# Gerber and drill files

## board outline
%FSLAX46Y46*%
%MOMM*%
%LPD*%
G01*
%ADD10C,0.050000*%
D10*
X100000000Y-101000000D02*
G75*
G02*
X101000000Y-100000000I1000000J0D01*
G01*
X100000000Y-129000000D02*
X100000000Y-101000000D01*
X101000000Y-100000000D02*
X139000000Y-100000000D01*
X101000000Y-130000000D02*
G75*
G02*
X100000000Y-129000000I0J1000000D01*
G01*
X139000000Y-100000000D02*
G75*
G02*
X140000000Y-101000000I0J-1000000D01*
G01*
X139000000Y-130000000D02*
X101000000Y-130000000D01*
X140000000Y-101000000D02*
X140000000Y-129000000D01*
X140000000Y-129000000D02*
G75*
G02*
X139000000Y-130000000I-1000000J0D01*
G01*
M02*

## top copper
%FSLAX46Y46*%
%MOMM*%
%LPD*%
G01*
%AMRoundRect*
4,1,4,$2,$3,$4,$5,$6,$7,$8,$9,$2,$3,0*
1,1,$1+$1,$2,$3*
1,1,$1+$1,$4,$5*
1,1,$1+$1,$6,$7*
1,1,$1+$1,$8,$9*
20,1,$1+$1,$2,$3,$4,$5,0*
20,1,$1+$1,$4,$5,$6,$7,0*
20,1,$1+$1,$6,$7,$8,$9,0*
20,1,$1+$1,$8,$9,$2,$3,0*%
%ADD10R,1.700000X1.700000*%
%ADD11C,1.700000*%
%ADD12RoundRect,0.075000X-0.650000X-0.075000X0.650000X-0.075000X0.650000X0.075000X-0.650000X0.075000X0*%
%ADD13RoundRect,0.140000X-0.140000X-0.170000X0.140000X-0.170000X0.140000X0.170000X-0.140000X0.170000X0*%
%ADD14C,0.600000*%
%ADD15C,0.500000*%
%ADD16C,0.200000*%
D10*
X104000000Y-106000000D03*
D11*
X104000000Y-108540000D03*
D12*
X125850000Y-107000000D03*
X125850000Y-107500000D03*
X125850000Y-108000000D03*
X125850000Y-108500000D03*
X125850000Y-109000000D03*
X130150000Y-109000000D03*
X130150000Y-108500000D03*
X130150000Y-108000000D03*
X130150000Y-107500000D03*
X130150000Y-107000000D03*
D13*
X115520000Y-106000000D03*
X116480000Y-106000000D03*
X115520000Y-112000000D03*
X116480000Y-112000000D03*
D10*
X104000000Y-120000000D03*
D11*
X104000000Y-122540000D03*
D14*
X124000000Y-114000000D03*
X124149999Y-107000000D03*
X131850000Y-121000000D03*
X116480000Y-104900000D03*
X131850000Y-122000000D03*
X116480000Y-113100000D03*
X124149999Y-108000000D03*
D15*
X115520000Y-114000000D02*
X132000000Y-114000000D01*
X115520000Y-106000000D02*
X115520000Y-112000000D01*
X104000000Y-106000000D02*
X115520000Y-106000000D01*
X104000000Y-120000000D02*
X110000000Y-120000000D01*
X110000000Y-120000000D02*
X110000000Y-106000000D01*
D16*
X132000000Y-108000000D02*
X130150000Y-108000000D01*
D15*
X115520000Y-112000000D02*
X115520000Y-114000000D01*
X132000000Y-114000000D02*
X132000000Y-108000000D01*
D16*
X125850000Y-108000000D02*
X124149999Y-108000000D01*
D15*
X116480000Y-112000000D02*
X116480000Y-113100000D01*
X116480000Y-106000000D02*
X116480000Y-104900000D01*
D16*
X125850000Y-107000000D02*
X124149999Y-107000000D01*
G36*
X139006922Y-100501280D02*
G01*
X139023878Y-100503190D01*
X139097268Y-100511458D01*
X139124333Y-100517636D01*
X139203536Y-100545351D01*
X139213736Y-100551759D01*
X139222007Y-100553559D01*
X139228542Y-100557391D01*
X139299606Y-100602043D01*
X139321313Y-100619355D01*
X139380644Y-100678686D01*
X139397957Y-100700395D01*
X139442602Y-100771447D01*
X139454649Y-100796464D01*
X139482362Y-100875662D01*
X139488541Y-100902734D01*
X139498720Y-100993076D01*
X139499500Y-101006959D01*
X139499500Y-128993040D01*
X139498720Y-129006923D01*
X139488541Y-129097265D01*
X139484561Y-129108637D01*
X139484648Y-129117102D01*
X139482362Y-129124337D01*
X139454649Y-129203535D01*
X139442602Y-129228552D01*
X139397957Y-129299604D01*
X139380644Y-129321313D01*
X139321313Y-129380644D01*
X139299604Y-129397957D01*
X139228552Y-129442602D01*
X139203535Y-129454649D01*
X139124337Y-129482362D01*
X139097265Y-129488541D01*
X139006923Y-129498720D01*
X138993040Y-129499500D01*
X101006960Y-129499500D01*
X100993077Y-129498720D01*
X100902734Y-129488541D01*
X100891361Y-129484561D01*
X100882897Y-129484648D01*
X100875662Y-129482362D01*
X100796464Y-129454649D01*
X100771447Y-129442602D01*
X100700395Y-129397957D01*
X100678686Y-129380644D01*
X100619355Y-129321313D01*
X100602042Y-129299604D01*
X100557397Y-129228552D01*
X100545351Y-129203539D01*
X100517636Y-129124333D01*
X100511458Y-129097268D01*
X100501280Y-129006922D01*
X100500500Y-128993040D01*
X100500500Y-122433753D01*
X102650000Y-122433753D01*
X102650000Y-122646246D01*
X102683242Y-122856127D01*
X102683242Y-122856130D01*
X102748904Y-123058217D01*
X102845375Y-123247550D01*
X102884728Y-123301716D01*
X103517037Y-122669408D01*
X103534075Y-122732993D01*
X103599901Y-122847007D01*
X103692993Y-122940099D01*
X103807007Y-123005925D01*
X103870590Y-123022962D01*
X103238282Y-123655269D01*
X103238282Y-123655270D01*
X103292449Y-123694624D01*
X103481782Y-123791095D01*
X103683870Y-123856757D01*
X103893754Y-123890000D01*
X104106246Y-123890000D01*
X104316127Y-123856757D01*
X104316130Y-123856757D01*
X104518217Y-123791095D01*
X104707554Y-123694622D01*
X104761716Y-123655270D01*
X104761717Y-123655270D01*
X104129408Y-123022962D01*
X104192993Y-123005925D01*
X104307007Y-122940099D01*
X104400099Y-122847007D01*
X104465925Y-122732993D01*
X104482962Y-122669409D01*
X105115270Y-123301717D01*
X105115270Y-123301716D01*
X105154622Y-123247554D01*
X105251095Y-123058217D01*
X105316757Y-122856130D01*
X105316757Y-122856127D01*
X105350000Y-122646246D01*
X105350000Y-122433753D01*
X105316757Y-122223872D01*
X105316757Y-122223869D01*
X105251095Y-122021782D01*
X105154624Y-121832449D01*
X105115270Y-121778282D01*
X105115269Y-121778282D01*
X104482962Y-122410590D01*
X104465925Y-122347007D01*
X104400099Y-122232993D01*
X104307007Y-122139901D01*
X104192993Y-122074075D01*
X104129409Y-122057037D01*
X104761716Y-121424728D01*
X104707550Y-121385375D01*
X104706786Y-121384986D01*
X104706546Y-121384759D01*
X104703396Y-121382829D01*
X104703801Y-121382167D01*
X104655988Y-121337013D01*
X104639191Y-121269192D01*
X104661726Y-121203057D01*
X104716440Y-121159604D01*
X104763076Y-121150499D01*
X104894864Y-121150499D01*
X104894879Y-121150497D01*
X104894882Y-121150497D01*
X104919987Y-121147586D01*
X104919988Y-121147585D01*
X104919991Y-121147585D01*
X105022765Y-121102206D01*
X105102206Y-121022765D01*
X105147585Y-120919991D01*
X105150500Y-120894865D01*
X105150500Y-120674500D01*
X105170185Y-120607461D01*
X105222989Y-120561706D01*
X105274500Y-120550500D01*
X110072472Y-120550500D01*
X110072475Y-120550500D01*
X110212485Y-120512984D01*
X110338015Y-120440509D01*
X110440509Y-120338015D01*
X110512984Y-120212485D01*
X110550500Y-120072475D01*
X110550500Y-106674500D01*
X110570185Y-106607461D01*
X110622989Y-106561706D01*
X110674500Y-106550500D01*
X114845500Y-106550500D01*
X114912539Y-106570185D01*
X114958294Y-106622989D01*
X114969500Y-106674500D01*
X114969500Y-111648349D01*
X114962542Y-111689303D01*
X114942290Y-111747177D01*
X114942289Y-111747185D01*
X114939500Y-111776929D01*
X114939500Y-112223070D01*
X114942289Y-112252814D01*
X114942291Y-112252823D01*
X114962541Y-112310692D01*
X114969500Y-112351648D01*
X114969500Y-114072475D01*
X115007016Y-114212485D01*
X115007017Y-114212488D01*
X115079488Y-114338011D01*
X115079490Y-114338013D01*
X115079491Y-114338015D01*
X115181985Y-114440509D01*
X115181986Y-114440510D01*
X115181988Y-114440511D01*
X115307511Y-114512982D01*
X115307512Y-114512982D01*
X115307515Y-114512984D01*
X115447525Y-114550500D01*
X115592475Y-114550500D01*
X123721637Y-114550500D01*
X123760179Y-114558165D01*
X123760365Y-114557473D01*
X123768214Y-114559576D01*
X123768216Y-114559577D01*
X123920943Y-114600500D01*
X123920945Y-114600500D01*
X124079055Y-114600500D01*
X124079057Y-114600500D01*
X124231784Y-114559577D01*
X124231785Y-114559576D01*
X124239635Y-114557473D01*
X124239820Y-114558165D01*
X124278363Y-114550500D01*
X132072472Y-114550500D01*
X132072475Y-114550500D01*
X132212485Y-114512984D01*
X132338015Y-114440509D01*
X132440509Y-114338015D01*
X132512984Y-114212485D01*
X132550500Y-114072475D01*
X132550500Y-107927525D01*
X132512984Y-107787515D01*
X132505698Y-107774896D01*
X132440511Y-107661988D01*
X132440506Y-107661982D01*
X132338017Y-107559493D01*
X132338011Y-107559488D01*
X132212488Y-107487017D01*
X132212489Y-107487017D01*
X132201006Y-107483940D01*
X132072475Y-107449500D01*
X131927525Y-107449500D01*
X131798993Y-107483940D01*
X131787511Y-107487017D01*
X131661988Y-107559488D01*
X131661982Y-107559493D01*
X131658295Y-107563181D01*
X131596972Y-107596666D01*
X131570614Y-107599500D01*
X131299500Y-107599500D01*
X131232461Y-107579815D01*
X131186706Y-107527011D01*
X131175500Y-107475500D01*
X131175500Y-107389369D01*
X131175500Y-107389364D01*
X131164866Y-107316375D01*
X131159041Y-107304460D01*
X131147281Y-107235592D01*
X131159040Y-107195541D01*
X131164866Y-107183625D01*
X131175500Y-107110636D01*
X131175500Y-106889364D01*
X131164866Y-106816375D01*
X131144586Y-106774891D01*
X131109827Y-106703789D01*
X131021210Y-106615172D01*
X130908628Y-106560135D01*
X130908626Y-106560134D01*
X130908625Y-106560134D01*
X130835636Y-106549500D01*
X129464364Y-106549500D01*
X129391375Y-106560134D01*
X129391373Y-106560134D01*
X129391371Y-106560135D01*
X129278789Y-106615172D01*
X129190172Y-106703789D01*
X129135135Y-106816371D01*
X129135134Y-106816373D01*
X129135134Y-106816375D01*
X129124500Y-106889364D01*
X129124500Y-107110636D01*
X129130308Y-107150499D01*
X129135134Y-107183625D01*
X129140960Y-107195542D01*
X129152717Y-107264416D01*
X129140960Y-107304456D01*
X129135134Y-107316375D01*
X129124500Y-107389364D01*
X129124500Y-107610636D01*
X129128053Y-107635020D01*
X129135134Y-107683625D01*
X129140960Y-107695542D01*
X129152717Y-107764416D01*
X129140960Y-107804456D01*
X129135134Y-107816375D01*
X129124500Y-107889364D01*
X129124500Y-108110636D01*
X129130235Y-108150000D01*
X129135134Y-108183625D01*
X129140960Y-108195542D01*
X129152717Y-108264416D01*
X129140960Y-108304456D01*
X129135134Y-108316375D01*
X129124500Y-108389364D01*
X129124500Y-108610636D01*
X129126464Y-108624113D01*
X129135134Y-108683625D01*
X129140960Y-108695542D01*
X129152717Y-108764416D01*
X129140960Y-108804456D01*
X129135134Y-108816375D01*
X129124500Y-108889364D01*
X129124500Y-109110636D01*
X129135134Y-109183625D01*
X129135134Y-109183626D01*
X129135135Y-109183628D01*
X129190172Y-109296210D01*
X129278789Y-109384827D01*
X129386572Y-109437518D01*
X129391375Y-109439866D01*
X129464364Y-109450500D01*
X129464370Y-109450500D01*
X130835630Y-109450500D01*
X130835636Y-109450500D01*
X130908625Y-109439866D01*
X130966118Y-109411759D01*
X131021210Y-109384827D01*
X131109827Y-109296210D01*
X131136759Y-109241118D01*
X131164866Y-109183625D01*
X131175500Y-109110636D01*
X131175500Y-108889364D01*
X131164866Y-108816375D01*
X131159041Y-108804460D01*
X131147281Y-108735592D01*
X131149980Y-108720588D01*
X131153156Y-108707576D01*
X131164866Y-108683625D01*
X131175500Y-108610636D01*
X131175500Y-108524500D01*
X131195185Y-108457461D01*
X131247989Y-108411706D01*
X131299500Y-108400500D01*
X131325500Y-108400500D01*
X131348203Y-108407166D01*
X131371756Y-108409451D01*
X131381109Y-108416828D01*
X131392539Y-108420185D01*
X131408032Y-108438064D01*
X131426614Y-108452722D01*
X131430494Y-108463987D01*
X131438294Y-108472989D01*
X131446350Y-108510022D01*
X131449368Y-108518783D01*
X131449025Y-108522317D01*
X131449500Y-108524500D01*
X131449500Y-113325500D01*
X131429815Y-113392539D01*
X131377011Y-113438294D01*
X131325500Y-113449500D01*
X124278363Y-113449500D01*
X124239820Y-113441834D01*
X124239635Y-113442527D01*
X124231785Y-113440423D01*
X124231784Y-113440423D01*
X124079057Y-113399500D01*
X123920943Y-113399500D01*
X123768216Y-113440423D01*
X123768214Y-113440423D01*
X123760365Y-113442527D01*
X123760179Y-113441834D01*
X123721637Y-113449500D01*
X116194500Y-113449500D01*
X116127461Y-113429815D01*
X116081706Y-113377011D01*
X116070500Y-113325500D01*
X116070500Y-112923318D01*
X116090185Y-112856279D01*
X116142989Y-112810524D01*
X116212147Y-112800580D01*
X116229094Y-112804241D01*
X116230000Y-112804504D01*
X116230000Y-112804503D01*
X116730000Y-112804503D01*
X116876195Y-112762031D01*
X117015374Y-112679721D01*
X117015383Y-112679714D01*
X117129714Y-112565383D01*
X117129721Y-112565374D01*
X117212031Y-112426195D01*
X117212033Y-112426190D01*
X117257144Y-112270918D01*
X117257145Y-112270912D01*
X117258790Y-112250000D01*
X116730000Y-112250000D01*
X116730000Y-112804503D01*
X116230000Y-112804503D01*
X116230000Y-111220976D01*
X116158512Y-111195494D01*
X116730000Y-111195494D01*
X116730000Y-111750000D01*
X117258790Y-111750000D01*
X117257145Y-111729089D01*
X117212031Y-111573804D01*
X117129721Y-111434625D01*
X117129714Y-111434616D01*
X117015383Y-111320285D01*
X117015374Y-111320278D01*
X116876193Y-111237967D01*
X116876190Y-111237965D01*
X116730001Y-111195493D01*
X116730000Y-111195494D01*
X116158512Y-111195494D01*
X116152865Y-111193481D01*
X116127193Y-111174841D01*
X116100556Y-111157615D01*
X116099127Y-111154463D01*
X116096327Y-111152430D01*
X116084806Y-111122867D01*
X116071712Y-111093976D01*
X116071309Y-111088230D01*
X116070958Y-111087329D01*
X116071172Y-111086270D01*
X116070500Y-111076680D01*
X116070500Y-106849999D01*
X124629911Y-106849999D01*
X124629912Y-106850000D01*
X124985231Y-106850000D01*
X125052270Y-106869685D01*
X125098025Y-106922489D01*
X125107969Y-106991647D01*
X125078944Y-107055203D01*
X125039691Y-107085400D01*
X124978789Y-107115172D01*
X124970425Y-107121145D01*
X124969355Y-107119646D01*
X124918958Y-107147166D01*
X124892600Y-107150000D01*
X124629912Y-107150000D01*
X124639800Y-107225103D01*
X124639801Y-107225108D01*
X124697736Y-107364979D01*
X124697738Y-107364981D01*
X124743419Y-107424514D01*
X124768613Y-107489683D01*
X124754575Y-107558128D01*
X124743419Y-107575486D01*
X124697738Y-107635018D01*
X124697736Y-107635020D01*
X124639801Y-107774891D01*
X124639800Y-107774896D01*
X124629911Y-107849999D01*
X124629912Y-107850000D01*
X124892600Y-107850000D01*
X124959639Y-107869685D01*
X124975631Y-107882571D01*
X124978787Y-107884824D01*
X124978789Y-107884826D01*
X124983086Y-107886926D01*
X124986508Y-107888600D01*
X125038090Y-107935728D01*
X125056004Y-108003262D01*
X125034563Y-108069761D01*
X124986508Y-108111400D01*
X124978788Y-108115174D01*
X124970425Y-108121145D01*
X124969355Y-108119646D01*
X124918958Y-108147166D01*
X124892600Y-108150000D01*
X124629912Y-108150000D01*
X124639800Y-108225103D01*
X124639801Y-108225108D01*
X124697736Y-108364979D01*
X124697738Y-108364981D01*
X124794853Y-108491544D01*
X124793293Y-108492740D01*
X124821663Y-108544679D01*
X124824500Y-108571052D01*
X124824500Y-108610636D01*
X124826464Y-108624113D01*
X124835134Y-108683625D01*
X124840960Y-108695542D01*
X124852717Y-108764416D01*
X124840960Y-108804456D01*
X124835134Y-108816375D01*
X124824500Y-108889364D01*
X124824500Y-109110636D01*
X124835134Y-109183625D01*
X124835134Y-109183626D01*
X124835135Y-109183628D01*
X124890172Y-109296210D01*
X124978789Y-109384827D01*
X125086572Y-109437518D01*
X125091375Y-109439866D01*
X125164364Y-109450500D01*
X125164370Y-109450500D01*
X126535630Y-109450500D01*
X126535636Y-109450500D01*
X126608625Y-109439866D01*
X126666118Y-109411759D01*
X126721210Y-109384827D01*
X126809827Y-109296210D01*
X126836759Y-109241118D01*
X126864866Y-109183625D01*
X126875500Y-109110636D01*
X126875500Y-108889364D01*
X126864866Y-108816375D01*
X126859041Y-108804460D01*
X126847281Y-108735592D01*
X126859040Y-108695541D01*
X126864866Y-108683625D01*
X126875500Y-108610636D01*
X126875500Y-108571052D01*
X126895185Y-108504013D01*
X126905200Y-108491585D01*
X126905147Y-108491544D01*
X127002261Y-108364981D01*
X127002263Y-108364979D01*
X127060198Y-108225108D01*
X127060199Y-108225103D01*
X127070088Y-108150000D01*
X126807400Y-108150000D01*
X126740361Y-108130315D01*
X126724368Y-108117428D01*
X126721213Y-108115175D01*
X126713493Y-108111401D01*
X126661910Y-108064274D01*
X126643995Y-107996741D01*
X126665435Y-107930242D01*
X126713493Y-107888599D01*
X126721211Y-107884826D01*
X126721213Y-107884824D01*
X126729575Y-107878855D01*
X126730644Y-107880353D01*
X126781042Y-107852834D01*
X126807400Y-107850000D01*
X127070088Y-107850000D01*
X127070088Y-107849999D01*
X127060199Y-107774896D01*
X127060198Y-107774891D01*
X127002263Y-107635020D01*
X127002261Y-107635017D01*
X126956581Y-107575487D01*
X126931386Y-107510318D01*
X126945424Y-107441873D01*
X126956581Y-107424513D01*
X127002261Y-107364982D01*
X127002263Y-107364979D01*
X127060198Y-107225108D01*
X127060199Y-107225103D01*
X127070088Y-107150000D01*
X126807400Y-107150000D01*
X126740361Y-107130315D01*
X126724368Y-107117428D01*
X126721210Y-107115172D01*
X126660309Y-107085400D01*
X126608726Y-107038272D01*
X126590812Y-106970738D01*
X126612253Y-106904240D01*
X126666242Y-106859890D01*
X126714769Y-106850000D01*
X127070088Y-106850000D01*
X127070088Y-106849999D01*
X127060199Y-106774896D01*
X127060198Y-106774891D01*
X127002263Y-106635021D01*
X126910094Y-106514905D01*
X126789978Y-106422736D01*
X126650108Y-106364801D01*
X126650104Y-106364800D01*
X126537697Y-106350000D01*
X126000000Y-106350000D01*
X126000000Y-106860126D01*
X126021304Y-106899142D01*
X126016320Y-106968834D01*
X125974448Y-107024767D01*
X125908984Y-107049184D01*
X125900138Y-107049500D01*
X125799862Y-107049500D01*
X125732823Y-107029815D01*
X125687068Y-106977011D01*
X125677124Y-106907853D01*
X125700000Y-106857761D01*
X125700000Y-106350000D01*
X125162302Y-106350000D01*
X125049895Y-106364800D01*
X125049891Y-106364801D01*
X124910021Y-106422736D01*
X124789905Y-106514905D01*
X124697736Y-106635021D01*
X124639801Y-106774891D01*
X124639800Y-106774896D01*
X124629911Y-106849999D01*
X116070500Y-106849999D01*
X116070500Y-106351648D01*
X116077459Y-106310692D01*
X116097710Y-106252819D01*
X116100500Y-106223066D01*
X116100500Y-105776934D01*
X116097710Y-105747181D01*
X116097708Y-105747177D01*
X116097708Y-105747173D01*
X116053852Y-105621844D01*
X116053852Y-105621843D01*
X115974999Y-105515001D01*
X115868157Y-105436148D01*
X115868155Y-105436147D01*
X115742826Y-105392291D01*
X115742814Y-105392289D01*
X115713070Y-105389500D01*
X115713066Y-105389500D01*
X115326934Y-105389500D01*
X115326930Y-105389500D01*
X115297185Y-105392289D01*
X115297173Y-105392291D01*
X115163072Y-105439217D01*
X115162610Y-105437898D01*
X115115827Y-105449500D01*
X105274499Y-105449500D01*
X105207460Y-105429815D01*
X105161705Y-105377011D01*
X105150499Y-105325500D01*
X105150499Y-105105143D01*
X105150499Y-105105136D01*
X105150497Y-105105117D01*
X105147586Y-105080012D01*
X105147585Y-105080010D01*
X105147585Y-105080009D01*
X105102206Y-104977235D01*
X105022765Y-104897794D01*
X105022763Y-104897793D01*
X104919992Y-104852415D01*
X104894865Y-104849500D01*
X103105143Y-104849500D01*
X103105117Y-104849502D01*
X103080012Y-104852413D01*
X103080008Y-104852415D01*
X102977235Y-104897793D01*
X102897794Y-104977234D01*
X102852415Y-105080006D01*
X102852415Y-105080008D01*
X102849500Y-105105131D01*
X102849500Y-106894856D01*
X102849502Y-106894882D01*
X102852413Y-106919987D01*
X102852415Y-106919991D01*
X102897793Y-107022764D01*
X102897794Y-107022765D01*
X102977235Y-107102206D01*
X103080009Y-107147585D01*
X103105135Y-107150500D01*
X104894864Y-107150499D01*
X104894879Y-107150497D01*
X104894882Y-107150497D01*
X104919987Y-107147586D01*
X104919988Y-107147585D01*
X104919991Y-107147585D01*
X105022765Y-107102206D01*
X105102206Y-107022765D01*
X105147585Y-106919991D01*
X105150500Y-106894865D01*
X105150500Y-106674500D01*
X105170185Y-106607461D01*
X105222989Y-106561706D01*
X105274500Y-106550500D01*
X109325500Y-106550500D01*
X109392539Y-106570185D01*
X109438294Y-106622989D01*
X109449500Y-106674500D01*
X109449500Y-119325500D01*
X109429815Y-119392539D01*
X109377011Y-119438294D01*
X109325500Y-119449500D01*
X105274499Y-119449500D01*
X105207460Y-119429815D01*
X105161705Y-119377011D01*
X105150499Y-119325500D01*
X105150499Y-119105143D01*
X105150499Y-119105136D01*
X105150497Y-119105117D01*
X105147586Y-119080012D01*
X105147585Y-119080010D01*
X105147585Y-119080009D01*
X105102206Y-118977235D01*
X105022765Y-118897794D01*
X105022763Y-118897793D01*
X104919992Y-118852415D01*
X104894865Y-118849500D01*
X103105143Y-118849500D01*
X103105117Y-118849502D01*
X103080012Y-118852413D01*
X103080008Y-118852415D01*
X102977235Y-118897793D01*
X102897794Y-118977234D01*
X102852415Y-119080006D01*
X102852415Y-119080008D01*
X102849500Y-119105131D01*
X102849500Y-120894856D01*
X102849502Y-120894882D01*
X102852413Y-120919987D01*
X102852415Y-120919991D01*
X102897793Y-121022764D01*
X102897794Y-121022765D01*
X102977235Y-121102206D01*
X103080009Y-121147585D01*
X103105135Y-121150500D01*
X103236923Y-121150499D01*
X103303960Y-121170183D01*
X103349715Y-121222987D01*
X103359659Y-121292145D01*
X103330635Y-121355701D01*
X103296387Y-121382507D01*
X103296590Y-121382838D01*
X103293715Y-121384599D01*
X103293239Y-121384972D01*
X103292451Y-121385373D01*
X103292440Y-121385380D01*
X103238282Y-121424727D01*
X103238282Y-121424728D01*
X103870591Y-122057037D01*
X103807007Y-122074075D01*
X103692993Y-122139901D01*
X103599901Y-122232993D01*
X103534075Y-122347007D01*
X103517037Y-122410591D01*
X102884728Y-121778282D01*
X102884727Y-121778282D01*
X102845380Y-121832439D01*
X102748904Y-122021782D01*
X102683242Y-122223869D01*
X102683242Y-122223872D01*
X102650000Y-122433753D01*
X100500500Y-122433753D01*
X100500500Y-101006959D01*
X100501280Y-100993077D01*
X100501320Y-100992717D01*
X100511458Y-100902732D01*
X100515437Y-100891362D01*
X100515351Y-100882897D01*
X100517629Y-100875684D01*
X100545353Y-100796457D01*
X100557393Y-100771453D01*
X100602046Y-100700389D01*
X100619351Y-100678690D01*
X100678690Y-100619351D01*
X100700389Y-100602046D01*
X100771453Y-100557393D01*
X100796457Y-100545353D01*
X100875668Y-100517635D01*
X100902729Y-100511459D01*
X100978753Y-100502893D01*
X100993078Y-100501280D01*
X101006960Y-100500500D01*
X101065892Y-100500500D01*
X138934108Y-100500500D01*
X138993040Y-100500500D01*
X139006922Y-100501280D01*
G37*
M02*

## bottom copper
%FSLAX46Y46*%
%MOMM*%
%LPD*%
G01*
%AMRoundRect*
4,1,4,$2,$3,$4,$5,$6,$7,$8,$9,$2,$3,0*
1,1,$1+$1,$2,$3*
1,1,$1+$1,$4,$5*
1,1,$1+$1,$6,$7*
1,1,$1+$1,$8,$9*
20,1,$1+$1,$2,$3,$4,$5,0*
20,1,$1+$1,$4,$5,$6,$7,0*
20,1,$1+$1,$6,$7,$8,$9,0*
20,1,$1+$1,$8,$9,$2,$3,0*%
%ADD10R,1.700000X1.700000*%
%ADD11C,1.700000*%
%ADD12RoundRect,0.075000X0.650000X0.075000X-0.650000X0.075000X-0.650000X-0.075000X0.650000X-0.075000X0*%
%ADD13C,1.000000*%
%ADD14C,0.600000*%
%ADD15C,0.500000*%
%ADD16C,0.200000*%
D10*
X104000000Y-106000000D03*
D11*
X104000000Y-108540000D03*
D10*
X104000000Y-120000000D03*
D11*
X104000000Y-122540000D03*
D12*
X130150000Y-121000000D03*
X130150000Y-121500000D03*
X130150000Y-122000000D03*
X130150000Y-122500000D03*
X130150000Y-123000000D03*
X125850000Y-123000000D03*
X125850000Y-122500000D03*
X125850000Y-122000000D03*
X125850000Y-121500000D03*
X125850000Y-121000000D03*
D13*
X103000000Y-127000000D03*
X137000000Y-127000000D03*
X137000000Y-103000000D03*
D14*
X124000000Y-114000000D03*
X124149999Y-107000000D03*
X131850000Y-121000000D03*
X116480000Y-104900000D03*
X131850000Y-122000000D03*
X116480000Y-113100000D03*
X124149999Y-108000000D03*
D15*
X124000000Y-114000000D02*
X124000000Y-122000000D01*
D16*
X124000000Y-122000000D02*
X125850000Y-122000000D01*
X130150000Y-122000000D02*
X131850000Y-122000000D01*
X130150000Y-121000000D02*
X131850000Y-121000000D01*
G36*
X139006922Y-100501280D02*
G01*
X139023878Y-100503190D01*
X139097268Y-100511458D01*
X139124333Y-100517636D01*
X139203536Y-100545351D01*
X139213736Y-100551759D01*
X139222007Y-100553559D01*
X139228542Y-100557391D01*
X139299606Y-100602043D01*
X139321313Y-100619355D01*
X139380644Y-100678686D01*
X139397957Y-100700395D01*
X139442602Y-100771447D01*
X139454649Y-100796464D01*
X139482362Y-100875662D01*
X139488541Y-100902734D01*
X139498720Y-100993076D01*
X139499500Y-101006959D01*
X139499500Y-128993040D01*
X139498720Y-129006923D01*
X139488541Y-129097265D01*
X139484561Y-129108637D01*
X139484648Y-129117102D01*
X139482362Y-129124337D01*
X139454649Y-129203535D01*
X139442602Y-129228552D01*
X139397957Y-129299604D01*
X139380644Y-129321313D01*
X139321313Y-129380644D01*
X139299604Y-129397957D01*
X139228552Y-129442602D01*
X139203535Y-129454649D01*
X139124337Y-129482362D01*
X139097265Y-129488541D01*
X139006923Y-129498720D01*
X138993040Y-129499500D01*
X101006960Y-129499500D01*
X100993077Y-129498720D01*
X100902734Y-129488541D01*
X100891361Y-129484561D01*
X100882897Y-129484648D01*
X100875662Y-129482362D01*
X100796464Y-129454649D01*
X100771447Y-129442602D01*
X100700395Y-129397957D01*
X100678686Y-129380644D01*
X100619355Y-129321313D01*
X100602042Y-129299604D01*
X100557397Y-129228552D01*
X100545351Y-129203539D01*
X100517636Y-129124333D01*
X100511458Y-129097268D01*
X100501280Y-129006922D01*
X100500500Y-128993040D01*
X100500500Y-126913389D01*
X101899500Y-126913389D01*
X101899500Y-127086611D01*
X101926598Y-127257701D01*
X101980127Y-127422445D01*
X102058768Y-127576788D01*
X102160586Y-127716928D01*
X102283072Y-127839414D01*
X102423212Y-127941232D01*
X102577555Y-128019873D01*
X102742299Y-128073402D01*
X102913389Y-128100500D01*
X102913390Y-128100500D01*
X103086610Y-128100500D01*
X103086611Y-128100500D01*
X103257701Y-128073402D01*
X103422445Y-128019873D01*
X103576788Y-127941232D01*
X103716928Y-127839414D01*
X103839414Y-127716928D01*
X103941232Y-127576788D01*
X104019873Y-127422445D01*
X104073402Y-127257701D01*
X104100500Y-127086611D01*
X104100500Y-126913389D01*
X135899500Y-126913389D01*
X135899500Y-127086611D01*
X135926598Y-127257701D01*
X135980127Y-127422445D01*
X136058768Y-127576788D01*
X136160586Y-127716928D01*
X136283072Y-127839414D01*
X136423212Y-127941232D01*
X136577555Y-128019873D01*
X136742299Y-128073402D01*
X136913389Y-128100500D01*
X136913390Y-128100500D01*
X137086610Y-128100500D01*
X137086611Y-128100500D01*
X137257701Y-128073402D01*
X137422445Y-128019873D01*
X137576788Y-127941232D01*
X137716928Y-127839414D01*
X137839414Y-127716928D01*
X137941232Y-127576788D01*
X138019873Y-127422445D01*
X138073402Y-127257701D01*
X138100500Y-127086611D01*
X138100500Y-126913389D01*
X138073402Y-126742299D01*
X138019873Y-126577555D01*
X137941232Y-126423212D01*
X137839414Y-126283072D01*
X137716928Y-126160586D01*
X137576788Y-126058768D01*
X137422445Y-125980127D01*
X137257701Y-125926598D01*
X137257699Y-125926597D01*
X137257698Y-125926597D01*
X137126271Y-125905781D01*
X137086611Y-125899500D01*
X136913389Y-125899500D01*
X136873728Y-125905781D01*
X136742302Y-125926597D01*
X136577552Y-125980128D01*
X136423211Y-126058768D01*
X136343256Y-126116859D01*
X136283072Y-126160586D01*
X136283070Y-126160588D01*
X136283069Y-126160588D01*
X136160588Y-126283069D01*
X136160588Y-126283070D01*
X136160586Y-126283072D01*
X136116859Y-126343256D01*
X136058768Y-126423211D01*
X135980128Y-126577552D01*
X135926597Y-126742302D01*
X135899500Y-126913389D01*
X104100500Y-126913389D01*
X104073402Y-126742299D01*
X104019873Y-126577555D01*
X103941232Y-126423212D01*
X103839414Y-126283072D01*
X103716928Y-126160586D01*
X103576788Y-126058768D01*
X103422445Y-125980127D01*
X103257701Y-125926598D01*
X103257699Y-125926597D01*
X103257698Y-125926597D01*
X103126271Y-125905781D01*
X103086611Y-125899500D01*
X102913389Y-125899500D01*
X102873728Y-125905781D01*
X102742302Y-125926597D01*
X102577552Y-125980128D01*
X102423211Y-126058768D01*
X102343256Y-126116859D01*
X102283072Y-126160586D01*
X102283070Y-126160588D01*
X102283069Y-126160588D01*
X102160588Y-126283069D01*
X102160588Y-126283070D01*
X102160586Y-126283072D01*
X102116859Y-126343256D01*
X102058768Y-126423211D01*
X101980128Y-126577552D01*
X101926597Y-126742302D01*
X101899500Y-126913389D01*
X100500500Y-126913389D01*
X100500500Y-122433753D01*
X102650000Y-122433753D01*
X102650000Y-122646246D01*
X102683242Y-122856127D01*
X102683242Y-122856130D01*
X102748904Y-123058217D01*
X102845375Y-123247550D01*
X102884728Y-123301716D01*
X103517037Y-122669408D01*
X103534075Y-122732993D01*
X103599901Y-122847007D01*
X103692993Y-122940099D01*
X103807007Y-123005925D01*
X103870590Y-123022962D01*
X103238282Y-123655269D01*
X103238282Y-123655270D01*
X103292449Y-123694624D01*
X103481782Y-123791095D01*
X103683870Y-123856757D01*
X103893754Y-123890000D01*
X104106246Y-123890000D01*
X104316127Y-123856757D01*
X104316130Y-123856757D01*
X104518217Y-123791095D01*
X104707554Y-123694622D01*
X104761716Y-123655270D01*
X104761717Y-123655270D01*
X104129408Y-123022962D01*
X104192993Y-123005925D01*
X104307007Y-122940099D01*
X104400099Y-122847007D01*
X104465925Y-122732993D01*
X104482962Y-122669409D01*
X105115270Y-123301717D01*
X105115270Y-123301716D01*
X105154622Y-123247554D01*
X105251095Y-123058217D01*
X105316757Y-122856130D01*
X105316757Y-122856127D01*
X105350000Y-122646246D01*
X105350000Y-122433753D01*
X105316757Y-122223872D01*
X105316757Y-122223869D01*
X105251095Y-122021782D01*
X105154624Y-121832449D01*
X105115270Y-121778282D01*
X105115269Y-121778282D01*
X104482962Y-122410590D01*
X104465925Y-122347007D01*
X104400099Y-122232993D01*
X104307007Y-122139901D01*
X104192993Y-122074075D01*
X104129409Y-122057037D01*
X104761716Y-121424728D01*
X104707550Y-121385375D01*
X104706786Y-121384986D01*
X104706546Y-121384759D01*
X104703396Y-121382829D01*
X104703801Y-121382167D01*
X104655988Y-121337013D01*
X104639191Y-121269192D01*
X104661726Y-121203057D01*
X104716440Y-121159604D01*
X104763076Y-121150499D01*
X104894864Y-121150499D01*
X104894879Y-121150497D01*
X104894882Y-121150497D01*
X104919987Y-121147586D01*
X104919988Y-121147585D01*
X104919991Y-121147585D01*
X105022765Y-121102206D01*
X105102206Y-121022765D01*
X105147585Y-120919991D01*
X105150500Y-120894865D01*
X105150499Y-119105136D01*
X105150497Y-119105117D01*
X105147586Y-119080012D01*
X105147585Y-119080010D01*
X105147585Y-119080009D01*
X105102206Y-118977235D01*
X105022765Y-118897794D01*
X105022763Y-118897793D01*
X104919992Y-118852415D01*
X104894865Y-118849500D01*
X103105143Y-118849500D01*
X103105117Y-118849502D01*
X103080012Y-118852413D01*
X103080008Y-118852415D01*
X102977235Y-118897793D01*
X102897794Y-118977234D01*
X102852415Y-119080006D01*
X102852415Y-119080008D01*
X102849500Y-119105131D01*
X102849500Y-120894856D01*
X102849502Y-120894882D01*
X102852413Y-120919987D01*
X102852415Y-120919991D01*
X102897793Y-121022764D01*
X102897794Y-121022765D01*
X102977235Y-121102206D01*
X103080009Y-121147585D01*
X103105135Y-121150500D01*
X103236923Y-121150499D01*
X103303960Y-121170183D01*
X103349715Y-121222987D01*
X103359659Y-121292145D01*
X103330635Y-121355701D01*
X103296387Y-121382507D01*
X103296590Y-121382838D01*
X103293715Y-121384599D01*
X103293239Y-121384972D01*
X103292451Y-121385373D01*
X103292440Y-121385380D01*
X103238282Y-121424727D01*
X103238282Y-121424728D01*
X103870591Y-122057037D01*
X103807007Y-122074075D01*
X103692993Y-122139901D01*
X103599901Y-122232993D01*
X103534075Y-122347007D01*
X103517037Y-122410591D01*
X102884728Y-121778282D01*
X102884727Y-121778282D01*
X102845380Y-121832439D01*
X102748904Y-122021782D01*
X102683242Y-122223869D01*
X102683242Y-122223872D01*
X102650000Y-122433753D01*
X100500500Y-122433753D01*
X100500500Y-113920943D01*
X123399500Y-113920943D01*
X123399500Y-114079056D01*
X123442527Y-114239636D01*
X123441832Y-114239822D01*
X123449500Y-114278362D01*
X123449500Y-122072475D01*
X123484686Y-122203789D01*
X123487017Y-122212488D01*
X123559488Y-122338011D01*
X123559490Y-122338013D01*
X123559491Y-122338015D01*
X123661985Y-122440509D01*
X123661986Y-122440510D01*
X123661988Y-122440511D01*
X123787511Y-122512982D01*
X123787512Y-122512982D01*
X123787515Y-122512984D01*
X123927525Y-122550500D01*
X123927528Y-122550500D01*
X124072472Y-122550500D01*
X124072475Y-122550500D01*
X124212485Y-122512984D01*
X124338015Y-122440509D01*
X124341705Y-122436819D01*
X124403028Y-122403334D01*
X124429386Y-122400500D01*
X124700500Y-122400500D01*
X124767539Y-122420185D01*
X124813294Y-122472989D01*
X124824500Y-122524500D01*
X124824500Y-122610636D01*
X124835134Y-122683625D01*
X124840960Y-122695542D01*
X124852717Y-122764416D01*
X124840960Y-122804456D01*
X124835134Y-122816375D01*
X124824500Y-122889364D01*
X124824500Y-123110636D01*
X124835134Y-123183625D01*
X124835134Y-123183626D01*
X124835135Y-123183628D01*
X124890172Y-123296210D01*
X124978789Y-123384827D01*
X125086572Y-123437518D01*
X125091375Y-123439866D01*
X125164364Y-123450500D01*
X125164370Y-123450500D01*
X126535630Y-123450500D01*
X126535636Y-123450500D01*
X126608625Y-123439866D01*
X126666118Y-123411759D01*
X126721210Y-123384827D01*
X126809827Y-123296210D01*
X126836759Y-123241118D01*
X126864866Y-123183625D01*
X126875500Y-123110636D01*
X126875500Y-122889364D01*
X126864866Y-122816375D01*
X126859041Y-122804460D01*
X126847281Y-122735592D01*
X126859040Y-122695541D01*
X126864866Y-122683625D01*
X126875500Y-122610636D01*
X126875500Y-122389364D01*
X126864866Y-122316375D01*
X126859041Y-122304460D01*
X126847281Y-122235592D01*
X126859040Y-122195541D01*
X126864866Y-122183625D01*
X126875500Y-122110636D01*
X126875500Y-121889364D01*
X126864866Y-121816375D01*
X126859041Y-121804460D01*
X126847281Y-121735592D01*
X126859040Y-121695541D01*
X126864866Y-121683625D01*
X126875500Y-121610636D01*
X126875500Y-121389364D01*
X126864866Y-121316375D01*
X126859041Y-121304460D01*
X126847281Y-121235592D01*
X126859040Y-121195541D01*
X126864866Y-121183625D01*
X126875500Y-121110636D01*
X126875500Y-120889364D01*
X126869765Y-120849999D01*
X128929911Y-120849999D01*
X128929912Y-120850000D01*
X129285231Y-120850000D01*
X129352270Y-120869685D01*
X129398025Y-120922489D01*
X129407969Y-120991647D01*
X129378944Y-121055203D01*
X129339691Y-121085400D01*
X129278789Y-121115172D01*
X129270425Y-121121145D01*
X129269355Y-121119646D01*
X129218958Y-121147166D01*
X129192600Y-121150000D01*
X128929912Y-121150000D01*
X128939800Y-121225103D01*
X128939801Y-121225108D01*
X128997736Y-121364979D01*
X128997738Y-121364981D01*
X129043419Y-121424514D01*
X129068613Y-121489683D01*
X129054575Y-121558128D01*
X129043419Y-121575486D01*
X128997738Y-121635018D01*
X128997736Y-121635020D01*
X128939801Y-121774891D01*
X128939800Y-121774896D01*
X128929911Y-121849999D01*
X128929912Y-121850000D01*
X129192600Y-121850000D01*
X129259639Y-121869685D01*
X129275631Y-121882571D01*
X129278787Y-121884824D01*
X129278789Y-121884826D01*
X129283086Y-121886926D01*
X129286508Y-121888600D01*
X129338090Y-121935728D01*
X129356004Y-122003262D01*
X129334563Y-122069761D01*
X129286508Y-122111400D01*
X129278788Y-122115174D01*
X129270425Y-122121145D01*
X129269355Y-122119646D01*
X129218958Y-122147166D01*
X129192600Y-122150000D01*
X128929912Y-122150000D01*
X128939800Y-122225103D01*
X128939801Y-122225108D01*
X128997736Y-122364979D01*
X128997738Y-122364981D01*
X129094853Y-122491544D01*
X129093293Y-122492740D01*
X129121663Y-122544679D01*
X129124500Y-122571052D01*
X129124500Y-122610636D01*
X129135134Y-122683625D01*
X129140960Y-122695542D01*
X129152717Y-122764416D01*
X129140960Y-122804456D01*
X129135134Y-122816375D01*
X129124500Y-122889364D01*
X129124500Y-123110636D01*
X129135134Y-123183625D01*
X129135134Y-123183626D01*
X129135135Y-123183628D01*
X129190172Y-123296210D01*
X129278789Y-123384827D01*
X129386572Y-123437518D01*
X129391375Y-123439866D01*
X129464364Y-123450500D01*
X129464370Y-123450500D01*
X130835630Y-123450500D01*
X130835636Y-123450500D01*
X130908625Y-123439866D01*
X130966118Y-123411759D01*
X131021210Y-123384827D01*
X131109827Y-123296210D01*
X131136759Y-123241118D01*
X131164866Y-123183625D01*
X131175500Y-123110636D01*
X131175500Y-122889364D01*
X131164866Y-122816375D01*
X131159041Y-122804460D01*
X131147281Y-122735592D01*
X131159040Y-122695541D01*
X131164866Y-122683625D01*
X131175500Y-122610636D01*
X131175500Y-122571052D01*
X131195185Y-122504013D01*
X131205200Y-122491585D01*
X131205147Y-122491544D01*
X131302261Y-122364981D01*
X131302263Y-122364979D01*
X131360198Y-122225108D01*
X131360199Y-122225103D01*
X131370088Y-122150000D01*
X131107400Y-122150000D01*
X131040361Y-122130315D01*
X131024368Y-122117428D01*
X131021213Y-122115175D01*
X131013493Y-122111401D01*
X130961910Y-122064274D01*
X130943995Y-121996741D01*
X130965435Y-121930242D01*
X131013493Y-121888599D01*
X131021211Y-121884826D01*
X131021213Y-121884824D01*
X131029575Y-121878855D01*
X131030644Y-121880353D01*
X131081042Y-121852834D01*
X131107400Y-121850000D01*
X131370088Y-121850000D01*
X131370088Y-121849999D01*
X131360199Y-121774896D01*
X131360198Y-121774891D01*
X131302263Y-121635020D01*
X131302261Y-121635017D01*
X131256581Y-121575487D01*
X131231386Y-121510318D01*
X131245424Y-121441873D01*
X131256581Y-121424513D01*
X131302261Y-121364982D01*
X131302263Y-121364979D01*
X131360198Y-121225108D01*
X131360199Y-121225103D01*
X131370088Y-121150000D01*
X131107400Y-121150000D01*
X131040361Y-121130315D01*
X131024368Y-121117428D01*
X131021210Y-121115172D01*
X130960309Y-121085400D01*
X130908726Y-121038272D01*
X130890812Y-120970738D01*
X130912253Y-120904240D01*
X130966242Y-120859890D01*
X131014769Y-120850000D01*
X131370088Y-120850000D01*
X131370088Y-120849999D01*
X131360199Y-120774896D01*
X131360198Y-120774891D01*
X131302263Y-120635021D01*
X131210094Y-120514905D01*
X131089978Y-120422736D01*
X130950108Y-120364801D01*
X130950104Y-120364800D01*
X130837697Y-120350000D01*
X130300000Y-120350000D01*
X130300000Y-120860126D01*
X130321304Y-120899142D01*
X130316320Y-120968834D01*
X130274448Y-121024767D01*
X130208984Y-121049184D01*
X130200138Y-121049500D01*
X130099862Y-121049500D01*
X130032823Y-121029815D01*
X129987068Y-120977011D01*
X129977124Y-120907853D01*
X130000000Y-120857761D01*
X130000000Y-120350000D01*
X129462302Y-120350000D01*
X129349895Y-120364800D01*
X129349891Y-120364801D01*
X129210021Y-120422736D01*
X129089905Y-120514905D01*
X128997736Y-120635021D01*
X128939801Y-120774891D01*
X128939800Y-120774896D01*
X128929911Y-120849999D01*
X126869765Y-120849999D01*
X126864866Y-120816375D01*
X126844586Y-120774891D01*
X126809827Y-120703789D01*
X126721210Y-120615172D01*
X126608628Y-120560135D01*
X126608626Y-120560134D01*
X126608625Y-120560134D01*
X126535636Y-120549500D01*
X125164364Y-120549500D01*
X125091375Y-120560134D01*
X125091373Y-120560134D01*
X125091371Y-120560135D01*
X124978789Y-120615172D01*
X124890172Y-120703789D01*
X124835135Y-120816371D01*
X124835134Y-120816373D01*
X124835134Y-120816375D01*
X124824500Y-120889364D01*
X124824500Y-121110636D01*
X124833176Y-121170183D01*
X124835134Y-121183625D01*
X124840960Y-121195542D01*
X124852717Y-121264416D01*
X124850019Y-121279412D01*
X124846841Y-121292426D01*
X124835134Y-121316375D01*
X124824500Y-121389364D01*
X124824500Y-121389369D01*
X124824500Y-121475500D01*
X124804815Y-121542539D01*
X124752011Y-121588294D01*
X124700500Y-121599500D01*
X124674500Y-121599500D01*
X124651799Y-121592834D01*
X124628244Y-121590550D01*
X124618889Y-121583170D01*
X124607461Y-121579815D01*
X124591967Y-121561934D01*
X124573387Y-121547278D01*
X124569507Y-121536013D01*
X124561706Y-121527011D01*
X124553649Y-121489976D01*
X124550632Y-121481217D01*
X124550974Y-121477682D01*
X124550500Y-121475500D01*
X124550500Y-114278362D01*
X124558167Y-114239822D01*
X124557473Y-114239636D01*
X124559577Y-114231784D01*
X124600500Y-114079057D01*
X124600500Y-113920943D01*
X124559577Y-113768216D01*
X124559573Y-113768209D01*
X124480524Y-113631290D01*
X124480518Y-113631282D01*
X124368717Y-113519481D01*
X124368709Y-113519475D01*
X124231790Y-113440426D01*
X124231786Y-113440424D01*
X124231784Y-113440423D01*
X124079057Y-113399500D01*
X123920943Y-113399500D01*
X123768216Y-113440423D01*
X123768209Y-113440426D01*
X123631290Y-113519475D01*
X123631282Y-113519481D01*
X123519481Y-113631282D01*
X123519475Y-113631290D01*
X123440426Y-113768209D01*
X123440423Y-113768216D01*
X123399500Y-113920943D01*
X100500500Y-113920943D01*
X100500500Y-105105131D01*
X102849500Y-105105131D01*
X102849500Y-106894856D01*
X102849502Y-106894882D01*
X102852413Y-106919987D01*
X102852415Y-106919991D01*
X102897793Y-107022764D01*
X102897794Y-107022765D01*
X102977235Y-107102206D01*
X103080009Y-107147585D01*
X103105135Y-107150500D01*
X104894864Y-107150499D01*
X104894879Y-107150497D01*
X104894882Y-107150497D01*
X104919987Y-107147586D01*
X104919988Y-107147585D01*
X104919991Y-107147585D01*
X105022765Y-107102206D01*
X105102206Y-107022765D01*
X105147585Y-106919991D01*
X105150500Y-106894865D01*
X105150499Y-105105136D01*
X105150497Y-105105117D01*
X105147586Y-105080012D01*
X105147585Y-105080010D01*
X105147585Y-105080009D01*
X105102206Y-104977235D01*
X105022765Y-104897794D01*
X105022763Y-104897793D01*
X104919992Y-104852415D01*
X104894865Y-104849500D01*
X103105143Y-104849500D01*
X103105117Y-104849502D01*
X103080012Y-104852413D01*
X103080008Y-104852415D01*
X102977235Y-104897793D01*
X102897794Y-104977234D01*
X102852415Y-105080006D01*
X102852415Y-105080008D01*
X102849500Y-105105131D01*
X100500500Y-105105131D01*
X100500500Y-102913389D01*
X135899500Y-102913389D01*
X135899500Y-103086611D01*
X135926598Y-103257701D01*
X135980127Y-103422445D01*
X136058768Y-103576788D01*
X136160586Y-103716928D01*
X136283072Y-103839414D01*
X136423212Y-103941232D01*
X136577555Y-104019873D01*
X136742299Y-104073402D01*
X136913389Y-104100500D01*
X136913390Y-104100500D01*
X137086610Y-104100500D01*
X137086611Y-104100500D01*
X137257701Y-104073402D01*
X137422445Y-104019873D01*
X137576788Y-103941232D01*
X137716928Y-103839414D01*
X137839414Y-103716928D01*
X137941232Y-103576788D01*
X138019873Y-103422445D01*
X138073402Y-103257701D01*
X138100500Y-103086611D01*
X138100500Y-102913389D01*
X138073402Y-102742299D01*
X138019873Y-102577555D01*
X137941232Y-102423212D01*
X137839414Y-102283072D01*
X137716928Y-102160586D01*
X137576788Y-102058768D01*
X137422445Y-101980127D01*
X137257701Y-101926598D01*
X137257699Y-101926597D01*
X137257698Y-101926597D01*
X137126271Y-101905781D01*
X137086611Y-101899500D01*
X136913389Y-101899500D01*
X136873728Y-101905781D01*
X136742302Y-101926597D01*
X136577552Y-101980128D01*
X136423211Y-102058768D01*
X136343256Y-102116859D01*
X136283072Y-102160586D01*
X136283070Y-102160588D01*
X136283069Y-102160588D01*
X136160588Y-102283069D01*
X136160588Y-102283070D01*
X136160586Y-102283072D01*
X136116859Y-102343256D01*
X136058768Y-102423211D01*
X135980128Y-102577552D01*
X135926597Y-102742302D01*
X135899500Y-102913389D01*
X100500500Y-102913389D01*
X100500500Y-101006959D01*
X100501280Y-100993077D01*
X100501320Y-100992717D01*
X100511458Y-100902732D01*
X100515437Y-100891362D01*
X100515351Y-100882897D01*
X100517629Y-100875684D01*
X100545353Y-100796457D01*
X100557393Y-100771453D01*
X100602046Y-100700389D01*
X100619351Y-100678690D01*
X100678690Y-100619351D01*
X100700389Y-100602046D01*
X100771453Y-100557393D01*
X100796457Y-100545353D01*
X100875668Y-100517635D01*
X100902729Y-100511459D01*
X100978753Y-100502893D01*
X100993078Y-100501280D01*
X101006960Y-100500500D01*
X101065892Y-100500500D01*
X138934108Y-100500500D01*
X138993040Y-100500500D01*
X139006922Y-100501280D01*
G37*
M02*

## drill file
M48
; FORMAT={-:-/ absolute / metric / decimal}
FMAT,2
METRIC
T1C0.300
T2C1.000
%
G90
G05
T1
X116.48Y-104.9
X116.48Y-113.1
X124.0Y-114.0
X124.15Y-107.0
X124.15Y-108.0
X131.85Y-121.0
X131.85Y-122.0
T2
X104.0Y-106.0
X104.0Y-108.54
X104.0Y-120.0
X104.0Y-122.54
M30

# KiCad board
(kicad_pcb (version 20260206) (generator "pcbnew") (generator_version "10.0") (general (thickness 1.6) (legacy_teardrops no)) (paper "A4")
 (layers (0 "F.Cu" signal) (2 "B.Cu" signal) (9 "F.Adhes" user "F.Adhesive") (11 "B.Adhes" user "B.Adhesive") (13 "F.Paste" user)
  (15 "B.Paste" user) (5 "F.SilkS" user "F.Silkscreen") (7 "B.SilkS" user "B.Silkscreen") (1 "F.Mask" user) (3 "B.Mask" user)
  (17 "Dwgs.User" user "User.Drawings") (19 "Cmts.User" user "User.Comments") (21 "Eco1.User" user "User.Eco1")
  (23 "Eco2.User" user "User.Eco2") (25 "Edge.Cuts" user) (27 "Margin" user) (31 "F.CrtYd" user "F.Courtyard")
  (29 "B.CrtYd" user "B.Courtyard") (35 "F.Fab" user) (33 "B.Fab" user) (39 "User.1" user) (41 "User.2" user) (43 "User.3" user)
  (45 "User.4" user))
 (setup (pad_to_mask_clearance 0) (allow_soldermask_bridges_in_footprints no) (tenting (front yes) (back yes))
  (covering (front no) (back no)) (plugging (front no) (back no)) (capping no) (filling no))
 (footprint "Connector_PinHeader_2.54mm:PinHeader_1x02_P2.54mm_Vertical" (layer "F.Cu") (at 104 106)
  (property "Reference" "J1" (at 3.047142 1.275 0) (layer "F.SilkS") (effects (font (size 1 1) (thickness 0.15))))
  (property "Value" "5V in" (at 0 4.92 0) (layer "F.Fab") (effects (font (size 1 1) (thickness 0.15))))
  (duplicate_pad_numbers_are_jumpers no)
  (pad "1" thru_hole rect (at 0 0) (size 1.7 1.7) (drill 1) (layers "*.Cu" "*.Mask") (remove_unused_layers no) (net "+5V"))
  (pad "2" thru_hole circle (at 0 2.54) (size 1.7 1.7) (drill 1) (layers "*.Cu" "*.Mask") (remove_unused_layers no) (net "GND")
   (zone_connect 2)))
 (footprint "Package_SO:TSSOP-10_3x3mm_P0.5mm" (layer "F.Cu") (at 128 108)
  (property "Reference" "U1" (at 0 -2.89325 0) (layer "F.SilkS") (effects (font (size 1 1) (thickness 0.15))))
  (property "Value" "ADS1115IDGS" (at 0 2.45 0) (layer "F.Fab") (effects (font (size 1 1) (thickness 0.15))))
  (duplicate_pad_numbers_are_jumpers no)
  (pad "1" smd roundrect (at -2.15 -1) (size 1.45 0.3) (layers "F.Cu" "F.Mask" "F.Paste") (roundrect_rratio 0.25) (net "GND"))
  (pad "2" smd roundrect (at -2.15 -0.5) (size 1.45 0.3) (layers "F.Cu" "F.Mask" "F.Paste") (roundrect_rratio 0.25)
   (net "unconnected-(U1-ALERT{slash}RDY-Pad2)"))
  (pad "3" smd roundrect (at -2.15 0) (size 1.45 0.3) (layers "F.Cu" "F.Mask" "F.Paste") (roundrect_rratio 0.25) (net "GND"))
  (pad "4" smd roundrect (at -2.15 0.5) (size 1.45 0.3) (layers "F.Cu" "F.Mask" "F.Paste") (roundrect_rratio 0.25)
   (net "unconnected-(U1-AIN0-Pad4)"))
  (pad "5" smd roundrect (at -2.15 1) (size 1.45 0.3) (layers "F.Cu" "F.Mask" "F.Paste") (roundrect_rratio 0.25)
   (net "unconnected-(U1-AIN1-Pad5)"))
  (pad "6" smd roundrect (at 2.15 1) (size 1.45 0.3) (layers "F.Cu" "F.Mask" "F.Paste") (roundrect_rratio 0.25)
   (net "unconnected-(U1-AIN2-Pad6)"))
  (pad "7" smd roundrect (at 2.15 0.5) (size 1.45 0.3) (layers "F.Cu" "F.Mask" "F.Paste") (roundrect_rratio 0.25)
   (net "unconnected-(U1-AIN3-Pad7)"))
  (pad "8" smd roundrect (at 2.15 0) (size 1.45 0.3) (layers "F.Cu" "F.Mask" "F.Paste") (roundrect_rratio 0.25) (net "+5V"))
  (pad "9" smd roundrect (at 2.15 -0.5) (size 1.45 0.3) (layers "F.Cu" "F.Mask" "F.Paste") (roundrect_rratio 0.25)
   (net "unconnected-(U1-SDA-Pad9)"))
  (pad "10" smd roundrect (at 2.15 -1) (size 1.45 0.3) (layers "F.Cu" "F.Mask" "F.Paste") (roundrect_rratio 0.25)
   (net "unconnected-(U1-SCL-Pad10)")))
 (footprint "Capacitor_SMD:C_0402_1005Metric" (layer "F.Cu") (at 116 106)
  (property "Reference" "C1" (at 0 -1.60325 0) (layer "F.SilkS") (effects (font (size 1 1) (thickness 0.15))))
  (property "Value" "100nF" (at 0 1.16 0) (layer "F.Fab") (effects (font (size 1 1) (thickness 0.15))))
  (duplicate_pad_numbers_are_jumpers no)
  (pad "1" smd roundrect (at -0.48 0) (size 0.56 0.62) (layers "F.Cu" "F.Mask" "F.Paste") (roundrect_rratio 0.25) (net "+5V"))
  (pad "2" smd roundrect (at 0.48 0) (size 0.56 0.62) (layers "F.Cu" "F.Mask" "F.Paste") (roundrect_rratio 0.25) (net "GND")
   (zone_connect 2)))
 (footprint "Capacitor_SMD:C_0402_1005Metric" (layer "F.Cu") (at 116 112)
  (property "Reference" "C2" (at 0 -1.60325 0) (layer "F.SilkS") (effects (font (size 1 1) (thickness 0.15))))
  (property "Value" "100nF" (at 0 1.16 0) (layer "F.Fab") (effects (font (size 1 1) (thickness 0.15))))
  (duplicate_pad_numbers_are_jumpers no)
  (pad "1" smd roundrect (at -0.48 0) (size 0.56 0.62) (layers "F.Cu" "F.Mask" "F.Paste") (roundrect_rratio 0.25) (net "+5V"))
  (pad "2" smd roundrect (at 0.48 0) (size 0.56 0.62) (layers "F.Cu" "F.Mask" "F.Paste") (roundrect_rratio 0.25) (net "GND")))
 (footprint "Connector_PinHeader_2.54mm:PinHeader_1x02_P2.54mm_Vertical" (layer "F.Cu") (at 104 120)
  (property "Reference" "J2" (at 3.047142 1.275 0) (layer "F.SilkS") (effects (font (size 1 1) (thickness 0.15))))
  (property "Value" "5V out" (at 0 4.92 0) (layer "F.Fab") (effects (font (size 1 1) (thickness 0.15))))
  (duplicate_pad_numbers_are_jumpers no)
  (pad "1" thru_hole rect (at 0 0) (size 1.7 1.7) (drill 1) (layers "*.Cu" "*.Mask") (remove_unused_layers no) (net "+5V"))
  (pad "2" thru_hole circle (at 0 2.54) (size 1.7 1.7) (drill 1) (layers "*.Cu" "*.Mask") (remove_unused_layers no) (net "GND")))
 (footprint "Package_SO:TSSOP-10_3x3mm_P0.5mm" (layer "B.Cu") (at 128 122 180)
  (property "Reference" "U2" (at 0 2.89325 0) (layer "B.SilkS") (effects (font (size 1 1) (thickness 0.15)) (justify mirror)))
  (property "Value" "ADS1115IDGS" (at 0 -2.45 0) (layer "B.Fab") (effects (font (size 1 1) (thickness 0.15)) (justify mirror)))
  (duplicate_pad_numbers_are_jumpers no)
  (pad "1" smd roundrect (at -2.15 1 180) (size 1.45 0.3) (layers "B.Cu" "B.Mask" "B.Paste") (roundrect_rratio 0.25) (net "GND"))
  (pad "2" smd roundrect (at -2.15 0.5 180) (size 1.45 0.3) (layers "B.Cu" "B.Mask" "B.Paste") (roundrect_rratio 0.25)
   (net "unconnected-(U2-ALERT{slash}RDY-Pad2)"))
  (pad "3" smd roundrect (at -2.15 0 180) (size 1.45 0.3) (layers "B.Cu" "B.Mask" "B.Paste") (roundrect_rratio 0.25) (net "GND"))
  (pad "4" smd roundrect (at -2.15 -0.5 180) (size 1.45 0.3) (layers "B.Cu" "B.Mask" "B.Paste") (roundrect_rratio 0.25)
   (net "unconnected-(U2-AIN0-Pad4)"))
  (pad "5" smd roundrect (at -2.15 -1 180) (size 1.45 0.3) (layers "B.Cu" "B.Mask" "B.Paste") (roundrect_rratio 0.25)
   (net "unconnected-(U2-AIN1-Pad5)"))
  (pad "6" smd roundrect (at 2.15 -1 180) (size 1.45 0.3) (layers "B.Cu" "B.Mask" "B.Paste") (roundrect_rratio 0.25)
   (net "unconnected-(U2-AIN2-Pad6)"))
  (pad "7" smd roundrect (at 2.15 -0.5 180) (size 1.45 0.3) (layers "B.Cu" "B.Mask" "B.Paste") (roundrect_rratio 0.25)
   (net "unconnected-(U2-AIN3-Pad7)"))
  (pad "8" smd roundrect (at 2.15 0 180) (size 1.45 0.3) (layers "B.Cu" "B.Mask" "B.Paste") (roundrect_rratio 0.25) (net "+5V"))
  (pad "9" smd roundrect (at 2.15 0.5 180) (size 1.45 0.3) (layers "B.Cu" "B.Mask" "B.Paste") (roundrect_rratio 0.25)
   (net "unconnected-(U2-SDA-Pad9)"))
  (pad "10" smd roundrect (at 2.15 1 180) (size 1.45 0.3) (layers "B.Cu" "B.Mask" "B.Paste") (roundrect_rratio 0.25)
   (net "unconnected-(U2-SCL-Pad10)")))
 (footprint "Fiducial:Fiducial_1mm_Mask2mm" (layer "B.Cu") (at 103 127 180)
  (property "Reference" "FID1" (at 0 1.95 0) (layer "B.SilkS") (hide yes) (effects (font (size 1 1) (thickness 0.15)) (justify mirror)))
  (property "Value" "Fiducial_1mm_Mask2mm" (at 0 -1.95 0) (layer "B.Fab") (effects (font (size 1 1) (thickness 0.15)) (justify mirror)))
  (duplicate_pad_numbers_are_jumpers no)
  (pad "" smd circle (at 0 0 180) (size 1 1) (layers "B.Cu" "B.Mask") (solder_mask_margin 0.5) (clearance 0.6)))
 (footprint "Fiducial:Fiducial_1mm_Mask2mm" (layer "B.Cu") (at 137 127 180)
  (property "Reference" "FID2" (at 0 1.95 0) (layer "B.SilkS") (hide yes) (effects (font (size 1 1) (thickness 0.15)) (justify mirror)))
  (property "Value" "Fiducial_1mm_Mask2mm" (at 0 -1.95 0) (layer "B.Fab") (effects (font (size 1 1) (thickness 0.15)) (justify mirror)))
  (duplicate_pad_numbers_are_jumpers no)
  (pad "" smd circle (at 0 0 180) (size 1 1) (layers "B.Cu" "B.Mask") (solder_mask_margin 0.5) (clearance 0.6)))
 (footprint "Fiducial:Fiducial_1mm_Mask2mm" (layer "B.Cu") (at 137 103 180)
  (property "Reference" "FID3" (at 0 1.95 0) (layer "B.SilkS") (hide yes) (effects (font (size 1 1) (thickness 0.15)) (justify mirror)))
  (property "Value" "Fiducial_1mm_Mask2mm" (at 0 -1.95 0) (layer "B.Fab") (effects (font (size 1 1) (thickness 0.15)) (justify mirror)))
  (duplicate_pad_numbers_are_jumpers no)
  (pad "" smd circle (at 0 0 180) (size 1 1) (layers "B.Cu" "B.Mask") (solder_mask_margin 0.5) (clearance 0.6)))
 (gr_arc (start 100 101) (mid 100.292893 100.292893) (end 101 100) (stroke (width 0.05) (type default)) (layer "Edge.Cuts"))
 (gr_line (start 100 129) (end 100 101) (stroke (width 0.05) (type default)) (layer "Edge.Cuts"))
 (gr_line (start 101 100) (end 139 100) (stroke (width 0.05) (type default)) (layer "Edge.Cuts"))
 (gr_arc (start 101 130) (mid 100.292893 129.707107) (end 100 129) (stroke (width 0.05) (type default)) (layer "Edge.Cuts"))
 (gr_arc (start 139 100) (mid 139.707107 100.292893) (end 140 101) (stroke (width 0.05) (type default)) (layer "Edge.Cuts"))
 (gr_line (start 139 130) (end 101 130) (stroke (width 0.05) (type default)) (layer "Edge.Cuts"))
 (gr_line (start 140 101) (end 140 129) (stroke (width 0.05) (type default)) (layer "Edge.Cuts"))
 (gr_arc (start 140 129) (mid 139.707107 129.707107) (end 139 130) (stroke (width 0.05) (type default)) (layer "Edge.Cuts"))
 (segment (start 115.52 114) (end 132 114) (width 0.5) (layer "F.Cu") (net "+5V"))
 (segment (start 115.52 106) (end 115.52 112) (width 0.5) (layer "F.Cu") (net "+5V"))
 (segment (start 104 106) (end 115.52 106) (width 0.5) (layer "F.Cu") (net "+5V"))
 (segment (start 104 120) (end 110 120) (width 0.5) (layer "F.Cu") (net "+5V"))
 (segment (start 110 120) (end 110 106) (width 0.5) (layer "F.Cu") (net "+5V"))
 (segment (start 132 108) (end 130.15 108) (width 0.2) (layer "F.Cu") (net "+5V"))
 (segment (start 115.52 112) (end 115.52 114) (width 0.5) (layer "F.Cu") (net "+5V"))
 (segment (start 132 114) (end 132 108) (width 0.5) (layer "F.Cu") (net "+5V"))
 (via (at 124 114) (size 0.6) (drill 0.3) (layers "F.Cu" "B.Cu") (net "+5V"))
 (segment (start 124 114) (end 124 122) (width 0.5) (layer "B.Cu") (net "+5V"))
 (segment (start 124 122) (end 125.85 122) (width 0.2) (layer "B.Cu") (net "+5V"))
 (segment (start 125.85 108) (end 124.149999 108) (width 0.2) (layer "F.Cu") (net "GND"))
 (segment (start 116.48 112) (end 116.48 113.1) (width 0.5) (layer "F.Cu") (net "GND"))
 (segment (start 116.48 106) (end 116.48 104.9) (width 0.5) (layer "F.Cu") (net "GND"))
 (segment (start 125.85 107) (end 124.149999 107) (width 0.2) (layer "F.Cu") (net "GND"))
 (via (at 124.149999 107) (size 0.6) (drill 0.3) (layers "F.Cu" "B.Cu") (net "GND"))
 (via (at 131.85 121) (size 0.6) (drill 0.3) (layers "F.Cu" "B.Cu") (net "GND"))
 (via (at 116.48 104.9) (size 0.6) (drill 0.3) (layers "F.Cu" "B.Cu") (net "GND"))
 (via (at 131.85 122) (size 0.6) (drill 0.3) (layers "F.Cu" "B.Cu") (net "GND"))
 (via (at 116.48 113.1) (size 0.6) (drill 0.3) (layers "F.Cu" "B.Cu") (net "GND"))
 (via (at 124.149999 108) (size 0.6) (drill 0.3) (layers "F.Cu" "B.Cu") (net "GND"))
 (segment (start 130.15 122) (end 131.85 122) (width 0.2) (layer "B.Cu") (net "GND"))
 (segment (start 130.15 121) (end 131.85 121) (width 0.2) (layer "B.Cu") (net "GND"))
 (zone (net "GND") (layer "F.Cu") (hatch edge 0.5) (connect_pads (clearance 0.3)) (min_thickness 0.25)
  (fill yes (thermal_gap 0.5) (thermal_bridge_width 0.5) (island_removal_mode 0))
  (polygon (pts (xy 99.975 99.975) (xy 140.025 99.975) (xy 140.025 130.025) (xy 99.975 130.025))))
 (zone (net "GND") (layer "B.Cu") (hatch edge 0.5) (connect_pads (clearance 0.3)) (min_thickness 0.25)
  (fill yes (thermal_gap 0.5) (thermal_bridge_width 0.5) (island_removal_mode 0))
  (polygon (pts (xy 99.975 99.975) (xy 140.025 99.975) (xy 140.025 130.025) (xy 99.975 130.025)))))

